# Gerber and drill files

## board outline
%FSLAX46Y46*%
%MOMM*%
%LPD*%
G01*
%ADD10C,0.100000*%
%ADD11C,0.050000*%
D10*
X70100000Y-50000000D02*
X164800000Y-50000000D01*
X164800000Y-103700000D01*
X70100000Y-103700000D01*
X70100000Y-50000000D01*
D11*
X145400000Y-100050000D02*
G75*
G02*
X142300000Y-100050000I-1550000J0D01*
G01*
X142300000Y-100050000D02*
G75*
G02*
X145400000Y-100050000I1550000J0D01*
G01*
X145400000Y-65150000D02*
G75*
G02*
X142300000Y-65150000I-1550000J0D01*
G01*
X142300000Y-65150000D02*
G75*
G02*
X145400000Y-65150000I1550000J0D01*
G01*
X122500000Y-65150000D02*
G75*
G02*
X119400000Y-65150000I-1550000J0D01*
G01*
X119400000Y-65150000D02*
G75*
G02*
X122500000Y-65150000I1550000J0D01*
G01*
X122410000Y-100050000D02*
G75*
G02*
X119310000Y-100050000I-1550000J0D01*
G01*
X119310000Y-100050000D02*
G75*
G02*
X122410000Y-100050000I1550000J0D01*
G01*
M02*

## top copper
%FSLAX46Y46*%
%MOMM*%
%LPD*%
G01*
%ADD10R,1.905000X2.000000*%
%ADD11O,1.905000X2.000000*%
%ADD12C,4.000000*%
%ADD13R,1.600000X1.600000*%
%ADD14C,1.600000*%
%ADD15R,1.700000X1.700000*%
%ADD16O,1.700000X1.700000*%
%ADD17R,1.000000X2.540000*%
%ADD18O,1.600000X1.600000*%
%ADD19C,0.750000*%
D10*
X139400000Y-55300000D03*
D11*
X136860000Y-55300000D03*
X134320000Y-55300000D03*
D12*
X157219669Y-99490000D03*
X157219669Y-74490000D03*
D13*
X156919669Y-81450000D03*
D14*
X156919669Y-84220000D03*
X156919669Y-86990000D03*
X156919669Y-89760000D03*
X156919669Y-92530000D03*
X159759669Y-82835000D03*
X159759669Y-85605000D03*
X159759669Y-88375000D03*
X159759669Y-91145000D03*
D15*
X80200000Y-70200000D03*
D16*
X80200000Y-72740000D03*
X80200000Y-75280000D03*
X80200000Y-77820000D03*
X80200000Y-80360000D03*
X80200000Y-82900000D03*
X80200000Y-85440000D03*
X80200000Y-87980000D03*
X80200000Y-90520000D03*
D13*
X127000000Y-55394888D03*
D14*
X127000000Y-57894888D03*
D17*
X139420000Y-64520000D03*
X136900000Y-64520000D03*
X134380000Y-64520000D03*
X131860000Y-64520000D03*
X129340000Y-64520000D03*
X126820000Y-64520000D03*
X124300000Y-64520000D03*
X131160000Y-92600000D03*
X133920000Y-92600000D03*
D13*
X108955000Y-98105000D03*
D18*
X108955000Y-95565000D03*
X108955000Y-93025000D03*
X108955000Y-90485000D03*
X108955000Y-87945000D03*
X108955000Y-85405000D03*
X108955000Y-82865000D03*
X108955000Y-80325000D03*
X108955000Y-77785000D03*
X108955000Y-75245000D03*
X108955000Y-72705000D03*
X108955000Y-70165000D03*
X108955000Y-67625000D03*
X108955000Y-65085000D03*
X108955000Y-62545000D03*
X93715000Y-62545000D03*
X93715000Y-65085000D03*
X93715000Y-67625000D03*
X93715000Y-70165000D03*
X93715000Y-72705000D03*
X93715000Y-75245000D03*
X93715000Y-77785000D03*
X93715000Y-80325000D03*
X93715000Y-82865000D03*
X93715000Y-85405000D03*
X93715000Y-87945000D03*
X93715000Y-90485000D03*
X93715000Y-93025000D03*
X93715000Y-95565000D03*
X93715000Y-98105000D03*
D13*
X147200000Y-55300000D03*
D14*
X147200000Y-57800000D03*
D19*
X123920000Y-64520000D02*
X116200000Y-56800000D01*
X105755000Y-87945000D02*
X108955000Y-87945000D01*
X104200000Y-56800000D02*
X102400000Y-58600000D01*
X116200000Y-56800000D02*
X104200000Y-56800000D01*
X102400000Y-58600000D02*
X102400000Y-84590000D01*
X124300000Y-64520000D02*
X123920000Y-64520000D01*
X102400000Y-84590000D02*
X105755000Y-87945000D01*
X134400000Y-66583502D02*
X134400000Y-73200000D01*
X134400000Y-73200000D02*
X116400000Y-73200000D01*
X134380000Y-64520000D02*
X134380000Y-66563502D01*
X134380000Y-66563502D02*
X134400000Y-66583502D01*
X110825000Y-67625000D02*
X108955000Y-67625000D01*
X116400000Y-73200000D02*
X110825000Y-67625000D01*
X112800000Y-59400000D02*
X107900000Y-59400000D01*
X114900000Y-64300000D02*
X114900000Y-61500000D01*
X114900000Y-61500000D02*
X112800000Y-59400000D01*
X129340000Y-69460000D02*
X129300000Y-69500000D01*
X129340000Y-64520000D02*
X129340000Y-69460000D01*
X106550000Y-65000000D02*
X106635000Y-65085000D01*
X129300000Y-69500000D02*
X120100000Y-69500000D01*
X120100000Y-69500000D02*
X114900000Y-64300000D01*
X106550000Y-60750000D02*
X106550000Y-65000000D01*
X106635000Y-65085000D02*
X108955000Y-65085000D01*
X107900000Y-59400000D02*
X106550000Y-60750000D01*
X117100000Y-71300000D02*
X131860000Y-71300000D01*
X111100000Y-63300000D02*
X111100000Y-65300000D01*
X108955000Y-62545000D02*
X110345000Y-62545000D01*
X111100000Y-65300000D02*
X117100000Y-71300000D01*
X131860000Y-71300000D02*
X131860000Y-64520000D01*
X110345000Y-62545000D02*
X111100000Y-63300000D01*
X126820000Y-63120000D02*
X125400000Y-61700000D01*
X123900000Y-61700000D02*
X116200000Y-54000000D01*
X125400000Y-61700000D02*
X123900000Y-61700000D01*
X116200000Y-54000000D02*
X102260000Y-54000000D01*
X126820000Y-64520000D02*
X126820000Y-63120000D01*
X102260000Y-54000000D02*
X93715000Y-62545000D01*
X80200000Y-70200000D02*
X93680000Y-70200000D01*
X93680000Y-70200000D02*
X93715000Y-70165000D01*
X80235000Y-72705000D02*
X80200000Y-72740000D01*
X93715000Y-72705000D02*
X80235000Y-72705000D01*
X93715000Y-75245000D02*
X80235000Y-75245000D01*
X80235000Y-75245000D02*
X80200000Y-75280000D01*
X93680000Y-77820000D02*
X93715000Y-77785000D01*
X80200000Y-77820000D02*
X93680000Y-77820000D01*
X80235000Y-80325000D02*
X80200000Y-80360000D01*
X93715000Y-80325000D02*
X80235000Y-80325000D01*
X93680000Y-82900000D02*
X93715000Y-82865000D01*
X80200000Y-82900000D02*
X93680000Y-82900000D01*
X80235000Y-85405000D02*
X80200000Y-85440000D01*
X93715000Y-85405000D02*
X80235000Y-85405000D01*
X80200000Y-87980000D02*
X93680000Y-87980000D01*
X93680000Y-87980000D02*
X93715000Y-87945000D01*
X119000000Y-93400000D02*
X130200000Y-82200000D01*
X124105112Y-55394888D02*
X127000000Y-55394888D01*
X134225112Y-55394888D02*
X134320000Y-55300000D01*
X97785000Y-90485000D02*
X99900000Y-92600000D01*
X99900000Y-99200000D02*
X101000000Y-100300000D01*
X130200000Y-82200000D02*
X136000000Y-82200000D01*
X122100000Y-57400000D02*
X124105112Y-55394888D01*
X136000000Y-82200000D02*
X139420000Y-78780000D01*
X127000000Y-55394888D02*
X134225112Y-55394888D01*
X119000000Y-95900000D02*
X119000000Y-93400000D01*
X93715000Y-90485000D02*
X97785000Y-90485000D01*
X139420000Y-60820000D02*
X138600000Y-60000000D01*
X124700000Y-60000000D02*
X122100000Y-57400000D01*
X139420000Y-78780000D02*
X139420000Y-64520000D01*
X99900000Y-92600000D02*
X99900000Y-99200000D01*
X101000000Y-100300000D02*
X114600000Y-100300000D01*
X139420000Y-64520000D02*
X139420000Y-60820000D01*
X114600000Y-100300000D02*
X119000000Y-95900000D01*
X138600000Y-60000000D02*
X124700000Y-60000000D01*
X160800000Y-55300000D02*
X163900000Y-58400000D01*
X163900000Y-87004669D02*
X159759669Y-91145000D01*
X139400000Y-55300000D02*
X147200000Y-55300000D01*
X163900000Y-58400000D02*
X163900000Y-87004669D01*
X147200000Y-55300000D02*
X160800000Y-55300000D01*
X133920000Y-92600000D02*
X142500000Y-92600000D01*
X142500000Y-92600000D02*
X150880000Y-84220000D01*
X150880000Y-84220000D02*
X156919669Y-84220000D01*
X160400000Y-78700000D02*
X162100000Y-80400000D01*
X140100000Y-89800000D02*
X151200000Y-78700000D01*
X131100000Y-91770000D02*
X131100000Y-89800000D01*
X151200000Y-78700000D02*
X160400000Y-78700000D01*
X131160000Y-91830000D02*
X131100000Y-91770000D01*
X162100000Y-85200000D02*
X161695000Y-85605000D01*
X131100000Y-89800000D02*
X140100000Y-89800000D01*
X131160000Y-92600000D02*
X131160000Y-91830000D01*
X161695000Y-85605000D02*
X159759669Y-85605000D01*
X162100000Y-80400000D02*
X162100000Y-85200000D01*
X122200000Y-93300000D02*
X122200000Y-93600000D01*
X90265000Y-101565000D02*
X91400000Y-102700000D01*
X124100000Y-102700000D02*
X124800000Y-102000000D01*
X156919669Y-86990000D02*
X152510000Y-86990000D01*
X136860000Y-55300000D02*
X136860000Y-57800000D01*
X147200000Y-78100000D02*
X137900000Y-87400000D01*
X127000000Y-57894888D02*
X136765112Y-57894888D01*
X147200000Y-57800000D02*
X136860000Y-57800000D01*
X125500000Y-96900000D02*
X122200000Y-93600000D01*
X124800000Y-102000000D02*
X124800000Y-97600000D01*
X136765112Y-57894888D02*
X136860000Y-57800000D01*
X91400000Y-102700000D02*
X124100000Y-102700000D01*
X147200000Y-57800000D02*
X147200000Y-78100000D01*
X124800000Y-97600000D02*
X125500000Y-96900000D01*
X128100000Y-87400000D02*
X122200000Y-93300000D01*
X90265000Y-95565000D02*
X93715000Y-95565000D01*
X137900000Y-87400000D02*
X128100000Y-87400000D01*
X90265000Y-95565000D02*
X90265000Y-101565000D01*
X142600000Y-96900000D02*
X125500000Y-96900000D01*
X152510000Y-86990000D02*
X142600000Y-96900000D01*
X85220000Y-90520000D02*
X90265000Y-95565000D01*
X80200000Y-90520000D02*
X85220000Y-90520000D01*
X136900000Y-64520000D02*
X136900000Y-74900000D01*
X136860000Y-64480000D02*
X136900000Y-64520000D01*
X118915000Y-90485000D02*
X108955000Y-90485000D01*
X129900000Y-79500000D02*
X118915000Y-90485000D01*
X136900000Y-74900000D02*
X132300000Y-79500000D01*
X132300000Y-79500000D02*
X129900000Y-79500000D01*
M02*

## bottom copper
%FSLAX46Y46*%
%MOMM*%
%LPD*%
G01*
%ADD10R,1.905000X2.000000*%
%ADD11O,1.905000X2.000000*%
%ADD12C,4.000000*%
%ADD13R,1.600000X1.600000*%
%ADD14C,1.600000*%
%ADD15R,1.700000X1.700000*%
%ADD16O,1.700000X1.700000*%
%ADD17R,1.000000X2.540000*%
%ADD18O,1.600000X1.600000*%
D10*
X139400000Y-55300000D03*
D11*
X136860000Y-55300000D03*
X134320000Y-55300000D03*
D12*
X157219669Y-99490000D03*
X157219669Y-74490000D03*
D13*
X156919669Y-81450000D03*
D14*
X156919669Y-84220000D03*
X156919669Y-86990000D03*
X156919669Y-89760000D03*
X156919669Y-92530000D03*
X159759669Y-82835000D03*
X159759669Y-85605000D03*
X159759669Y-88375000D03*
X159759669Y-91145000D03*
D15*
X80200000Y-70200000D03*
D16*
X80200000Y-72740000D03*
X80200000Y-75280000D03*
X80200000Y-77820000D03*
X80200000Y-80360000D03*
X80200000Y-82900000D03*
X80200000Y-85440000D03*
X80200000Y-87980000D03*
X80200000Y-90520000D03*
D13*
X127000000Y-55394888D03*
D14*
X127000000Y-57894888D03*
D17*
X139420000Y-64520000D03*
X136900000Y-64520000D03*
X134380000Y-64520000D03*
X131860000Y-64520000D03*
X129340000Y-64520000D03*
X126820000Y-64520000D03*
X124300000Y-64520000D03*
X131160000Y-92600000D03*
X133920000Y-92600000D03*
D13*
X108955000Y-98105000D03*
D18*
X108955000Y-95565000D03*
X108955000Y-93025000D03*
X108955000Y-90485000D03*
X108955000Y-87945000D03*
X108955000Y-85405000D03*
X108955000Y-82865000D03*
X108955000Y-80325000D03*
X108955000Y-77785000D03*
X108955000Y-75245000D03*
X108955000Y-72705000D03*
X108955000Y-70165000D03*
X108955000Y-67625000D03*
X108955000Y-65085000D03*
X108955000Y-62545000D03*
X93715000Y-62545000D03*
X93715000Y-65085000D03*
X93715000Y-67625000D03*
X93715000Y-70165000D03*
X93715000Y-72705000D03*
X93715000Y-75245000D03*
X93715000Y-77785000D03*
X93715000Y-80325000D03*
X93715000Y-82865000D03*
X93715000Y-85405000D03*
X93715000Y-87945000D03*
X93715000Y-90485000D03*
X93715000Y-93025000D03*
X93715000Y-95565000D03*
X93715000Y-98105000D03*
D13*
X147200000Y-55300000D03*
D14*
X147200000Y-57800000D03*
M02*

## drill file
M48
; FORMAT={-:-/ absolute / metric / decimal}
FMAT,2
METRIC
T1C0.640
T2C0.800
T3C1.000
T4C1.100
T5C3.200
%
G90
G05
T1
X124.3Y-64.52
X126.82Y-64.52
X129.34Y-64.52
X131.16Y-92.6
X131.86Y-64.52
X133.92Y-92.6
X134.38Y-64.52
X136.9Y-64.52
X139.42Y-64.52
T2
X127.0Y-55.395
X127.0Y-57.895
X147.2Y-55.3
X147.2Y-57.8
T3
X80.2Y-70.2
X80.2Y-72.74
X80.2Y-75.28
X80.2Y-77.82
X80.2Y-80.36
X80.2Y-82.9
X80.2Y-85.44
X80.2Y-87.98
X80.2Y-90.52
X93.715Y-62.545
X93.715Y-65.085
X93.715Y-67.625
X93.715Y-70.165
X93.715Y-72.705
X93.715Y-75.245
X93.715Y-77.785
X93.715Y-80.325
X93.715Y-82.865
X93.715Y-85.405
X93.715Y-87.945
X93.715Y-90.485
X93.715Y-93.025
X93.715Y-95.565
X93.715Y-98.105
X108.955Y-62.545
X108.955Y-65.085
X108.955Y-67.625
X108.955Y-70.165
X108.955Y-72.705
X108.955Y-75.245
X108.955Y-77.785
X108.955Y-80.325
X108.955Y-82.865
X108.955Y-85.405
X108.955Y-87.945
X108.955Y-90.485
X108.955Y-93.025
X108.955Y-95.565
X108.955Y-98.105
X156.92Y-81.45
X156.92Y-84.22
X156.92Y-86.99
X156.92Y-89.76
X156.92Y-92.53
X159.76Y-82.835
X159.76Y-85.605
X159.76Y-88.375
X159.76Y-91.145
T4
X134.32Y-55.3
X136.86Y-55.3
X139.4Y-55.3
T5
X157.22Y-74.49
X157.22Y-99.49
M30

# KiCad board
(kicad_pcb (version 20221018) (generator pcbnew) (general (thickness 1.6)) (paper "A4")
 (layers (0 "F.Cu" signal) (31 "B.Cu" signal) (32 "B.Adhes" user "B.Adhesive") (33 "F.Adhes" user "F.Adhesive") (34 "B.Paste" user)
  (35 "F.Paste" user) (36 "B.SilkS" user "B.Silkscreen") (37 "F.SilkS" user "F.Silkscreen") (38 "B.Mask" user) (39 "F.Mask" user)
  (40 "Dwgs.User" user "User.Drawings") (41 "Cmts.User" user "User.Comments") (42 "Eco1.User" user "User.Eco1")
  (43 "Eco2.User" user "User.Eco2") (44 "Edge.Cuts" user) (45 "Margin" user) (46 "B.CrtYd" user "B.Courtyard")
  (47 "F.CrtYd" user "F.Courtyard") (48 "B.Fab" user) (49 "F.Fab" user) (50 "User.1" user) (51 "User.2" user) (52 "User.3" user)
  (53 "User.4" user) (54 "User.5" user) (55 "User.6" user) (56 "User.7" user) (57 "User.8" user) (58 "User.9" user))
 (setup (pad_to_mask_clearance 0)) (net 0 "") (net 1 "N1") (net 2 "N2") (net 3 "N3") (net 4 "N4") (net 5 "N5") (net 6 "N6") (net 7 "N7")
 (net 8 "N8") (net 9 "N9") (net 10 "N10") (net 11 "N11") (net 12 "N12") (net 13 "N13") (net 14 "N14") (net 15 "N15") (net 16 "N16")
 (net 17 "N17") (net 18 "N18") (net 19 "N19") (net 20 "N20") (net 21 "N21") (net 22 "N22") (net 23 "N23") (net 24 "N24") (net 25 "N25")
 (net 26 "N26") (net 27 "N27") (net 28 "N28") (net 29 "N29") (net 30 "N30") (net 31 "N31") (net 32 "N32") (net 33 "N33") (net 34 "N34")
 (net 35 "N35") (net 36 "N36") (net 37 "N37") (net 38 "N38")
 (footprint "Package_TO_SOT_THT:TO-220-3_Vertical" (layer "F.Cu") (at 139.4 55.3 180)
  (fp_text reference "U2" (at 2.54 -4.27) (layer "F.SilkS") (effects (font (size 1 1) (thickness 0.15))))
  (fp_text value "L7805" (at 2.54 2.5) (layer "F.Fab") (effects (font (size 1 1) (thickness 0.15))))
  (pad "1" thru_hole rect (at 0 0 180) (size 1.905 2) (drill 1.1) (layers "*.Cu" "*.Mask") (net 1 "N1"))
  (pad "2" thru_hole oval (at 2.54 0 180) (size 1.905 2) (drill 1.1) (layers "*.Cu" "*.Mask") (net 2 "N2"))
  (pad "3" thru_hole oval (at 5.08 0 180) (size 1.905 2) (drill 1.1) (layers "*.Cu" "*.Mask") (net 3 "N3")))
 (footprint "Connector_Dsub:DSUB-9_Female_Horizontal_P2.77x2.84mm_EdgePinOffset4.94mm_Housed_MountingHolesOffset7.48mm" (layer "F.Cu")
  (at 156.919669 81.45 90)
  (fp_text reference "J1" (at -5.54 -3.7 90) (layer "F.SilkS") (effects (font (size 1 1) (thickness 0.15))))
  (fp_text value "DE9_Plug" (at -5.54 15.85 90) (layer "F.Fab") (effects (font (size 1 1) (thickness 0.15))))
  (pad "0" thru_hole circle (at -18.04 0.3 90) (size 4 4) (drill 3.2) (layers "*.Cu" "*.Mask"))
  (pad "0" thru_hole circle (at 6.96 0.3 90) (size 4 4) (drill 3.2) (layers "*.Cu" "*.Mask"))
  (pad "1" thru_hole rect (at 0 0 90) (size 1.6 1.6) (drill 1) (layers "*.Cu" "*.Mask") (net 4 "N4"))
  (pad "2" thru_hole circle (at -2.77 0 90) (size 1.6 1.6) (drill 1) (layers "*.Cu" "*.Mask") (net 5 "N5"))
  (pad "3" thru_hole circle (at -5.54 0 90) (size 1.6 1.6) (drill 1) (layers "*.Cu" "*.Mask") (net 2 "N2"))
  (pad "4" thru_hole circle (at -8.31 0 90) (size 1.6 1.6) (drill 1) (layers "*.Cu" "*.Mask") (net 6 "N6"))
  (pad "5" thru_hole circle (at -11.08 0 90) (size 1.6 1.6) (drill 1) (layers "*.Cu" "*.Mask") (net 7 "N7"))
  (pad "6" thru_hole circle (at -1.385 2.84 90) (size 1.6 1.6) (drill 1) (layers "*.Cu" "*.Mask") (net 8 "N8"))
  (pad "7" thru_hole circle (at -4.155 2.84 90) (size 1.6 1.6) (drill 1) (layers "*.Cu" "*.Mask") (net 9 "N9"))
  (pad "8" thru_hole circle (at -6.925 2.84 90) (size 1.6 1.6) (drill 1) (layers "*.Cu" "*.Mask") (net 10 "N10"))
  (pad "9" thru_hole circle (at -9.695 2.84 90) (size 1.6 1.6) (drill 1) (layers "*.Cu" "*.Mask") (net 1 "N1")))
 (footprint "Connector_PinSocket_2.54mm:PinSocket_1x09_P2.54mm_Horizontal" (layer "F.Cu") (at 80.2 70.2)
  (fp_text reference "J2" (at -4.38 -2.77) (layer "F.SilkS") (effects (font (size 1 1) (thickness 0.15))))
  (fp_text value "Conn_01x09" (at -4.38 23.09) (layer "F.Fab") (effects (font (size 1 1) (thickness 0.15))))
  (pad "1" thru_hole rect (at 0 0) (size 1.7 1.7) (drill 1) (layers "*.Cu" "*.Mask") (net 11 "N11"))
  (pad "2" thru_hole oval (at 0 2.54) (size 1.7 1.7) (drill 1) (layers "*.Cu" "*.Mask") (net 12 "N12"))
  (pad "3" thru_hole oval (at 0 5.08) (size 1.7 1.7) (drill 1) (layers "*.Cu" "*.Mask") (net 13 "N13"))
  (pad "4" thru_hole oval (at 0 7.62) (size 1.7 1.7) (drill 1) (layers "*.Cu" "*.Mask") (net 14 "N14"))
  (pad "5" thru_hole oval (at 0 10.16) (size 1.7 1.7) (drill 1) (layers "*.Cu" "*.Mask") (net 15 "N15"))
  (pad "6" thru_hole oval (at 0 12.7) (size 1.7 1.7) (drill 1) (layers "*.Cu" "*.Mask") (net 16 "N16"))
  (pad "7" thru_hole oval (at 0 15.24) (size 1.7 1.7) (drill 1) (layers "*.Cu" "*.Mask") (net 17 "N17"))
  (pad "8" thru_hole oval (at 0 17.78) (size 1.7 1.7) (drill 1) (layers "*.Cu" "*.Mask") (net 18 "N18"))
  (pad "9" thru_hole oval (at 0 20.32) (size 1.7 1.7) (drill 1) (layers "*.Cu" "*.Mask") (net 2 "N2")))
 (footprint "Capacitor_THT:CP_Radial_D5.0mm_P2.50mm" (layer "F.Cu") (at 127 55.394888 -90)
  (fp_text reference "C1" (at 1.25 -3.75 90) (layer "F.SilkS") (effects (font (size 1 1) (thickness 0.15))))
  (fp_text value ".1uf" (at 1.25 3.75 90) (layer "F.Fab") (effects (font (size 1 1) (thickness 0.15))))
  (pad "1" thru_hole rect (at 0 0 270) (size 1.6 1.6) (drill 0.8) (layers "*.Cu" "*.Mask") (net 3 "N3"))
  (pad "2" thru_hole circle (at 2.5 0 270) (size 1.6 1.6) (drill 0.8) (layers "*.Cu" "*.Mask") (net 2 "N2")))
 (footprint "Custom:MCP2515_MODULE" (layer "F.Cu") (at 118.3 62.6 180) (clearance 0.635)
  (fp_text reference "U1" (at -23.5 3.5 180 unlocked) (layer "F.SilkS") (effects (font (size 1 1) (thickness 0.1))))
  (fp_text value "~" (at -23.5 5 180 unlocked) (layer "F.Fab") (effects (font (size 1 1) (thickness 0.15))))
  (fp_circle (center -25.55 -37.45) (end -24 -37.45) (stroke (width 0.05) (type default)) (fill none) (layer "Edge.Cuts"))
  (fp_circle (center -25.55 -2.55) (end -24 -2.55) (stroke (width 0.05) (type default)) (fill none) (layer "Edge.Cuts"))
  (fp_circle (center -2.65 -2.55) (end -1.1 -2.55) (stroke (width 0.05) (type default)) (fill none) (layer "Edge.Cuts"))
  (fp_circle (center -2.56 -37.45) (end -1.01 -37.45) (stroke (width 0.05) (type default)) (fill none) (layer "Edge.Cuts"))
  (pad "1" thru_hole rect (at -21.12 -1.92 180) (size 1 2.54) (drill 0.64) (layers "*.Cu" "*.Mask") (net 3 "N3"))
  (pad "2" thru_hole rect (at -18.6 -1.92 180) (size 1 2.54) (drill 0.64) (layers "*.Cu" "*.Mask") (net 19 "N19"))
  (pad "3" thru_hole rect (at -16.08 -1.92 180) (size 1 2.54) (drill 0.64) (layers "*.Cu" "*.Mask") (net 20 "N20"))
  (pad "4" thru_hole rect (at -13.56 -1.92 180) (size 1 2.54) (drill 0.64) (layers "*.Cu" "*.Mask") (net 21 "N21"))
  (pad "5" thru_hole rect (at -11.04 -1.92 180) (size 1 2.54) (drill 0.64) (layers "*.Cu" "*.Mask") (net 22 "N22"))
  (pad "6" thru_hole rect (at -8.52 -1.92 180) (size 1 2.54) (drill 0.64) (layers "*.Cu" "*.Mask") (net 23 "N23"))
  (pad "7" thru_hole rect (at -6 -1.92 180) (size 1 2.54) (drill 0.64) (layers "*.Cu" "*.Mask") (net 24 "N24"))
  (pad "8" thru_hole rect (at -12.86 -30 180) (size 1 2.54) (drill 0.64) (layers "*.Cu" "*.Mask") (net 9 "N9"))
  (pad "9" thru_hole rect (at -15.62 -30 180) (size 1 2.54) (drill 0.64) (layers "*.Cu" "*.Mask") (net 5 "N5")))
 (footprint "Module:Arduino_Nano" (layer "F.Cu") (at 108.955 98.105 180)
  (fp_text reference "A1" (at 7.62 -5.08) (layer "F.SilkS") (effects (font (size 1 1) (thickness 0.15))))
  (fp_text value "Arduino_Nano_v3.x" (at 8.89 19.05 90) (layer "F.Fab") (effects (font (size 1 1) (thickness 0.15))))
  (pad "1" thru_hole rect (at 0 0 180) (size 1.6 1.6) (drill 1) (layers "*.Cu" "*.Mask") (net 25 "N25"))
  (pad "2" thru_hole oval (at 0 2.54 180) (size 1.6 1.6) (drill 1) (layers "*.Cu" "*.Mask") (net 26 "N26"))
  (pad "3" thru_hole oval (at 0 5.08 180) (size 1.6 1.6) (drill 1) (layers "*.Cu" "*.Mask") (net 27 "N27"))
  (pad "4" thru_hole oval (at 0 7.62 180) (size 1.6 1.6) (drill 1) (layers "*.Cu" "*.Mask") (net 19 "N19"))
  (pad "5" thru_hole oval (at 0 10.16 180) (size 1.6 1.6) (drill 1) (layers "*.Cu" "*.Mask") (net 24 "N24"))
  (pad "6" thru_hole oval (at 0 12.7 180) (size 1.6 1.6) (drill 1) (layers "*.Cu" "*.Mask") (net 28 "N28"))
  (pad "7" thru_hole oval (at 0 15.24 180) (size 1.6 1.6) (drill 1) (layers "*.Cu" "*.Mask") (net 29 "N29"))
  (pad "8" thru_hole oval (at 0 17.78 180) (size 1.6 1.6) (drill 1) (layers "*.Cu" "*.Mask") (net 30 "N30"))
  (pad "9" thru_hole oval (at 0 20.32 180) (size 1.6 1.6) (drill 1) (layers "*.Cu" "*.Mask") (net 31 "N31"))
  (pad "10" thru_hole oval (at 0 22.86 180) (size 1.6 1.6) (drill 1) (layers "*.Cu" "*.Mask") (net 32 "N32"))
  (pad "11" thru_hole oval (at 0 25.4 180) (size 1.6 1.6) (drill 1) (layers "*.Cu" "*.Mask") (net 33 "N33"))
  (pad "12" thru_hole oval (at 0 27.94 180) (size 1.6 1.6) (drill 1) (layers "*.Cu" "*.Mask") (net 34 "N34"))
  (pad "13" thru_hole oval (at 0 30.48 180) (size 1.6 1.6) (drill 1) (layers "*.Cu" "*.Mask") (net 20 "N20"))
  (pad "14" thru_hole oval (at 0 33.02 180) (size 1.6 1.6) (drill 1) (layers "*.Cu" "*.Mask") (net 22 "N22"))
  (pad "15" thru_hole oval (at 0 35.56 180) (size 1.6 1.6) (drill 1) (layers "*.Cu" "*.Mask") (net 21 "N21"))
  (pad "16" thru_hole oval (at 15.24 35.56 180) (size 1.6 1.6) (drill 1) (layers "*.Cu" "*.Mask") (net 23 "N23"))
  (pad "17" thru_hole oval (at 15.24 33.02 180) (size 1.6 1.6) (drill 1) (layers "*.Cu" "*.Mask") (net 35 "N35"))
  (pad "18" thru_hole oval (at 15.24 30.48 180) (size 1.6 1.6) (drill 1) (layers "*.Cu" "*.Mask") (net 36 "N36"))
  (pad "19" thru_hole oval (at 15.24 27.94 180) (size 1.6 1.6) (drill 1) (layers "*.Cu" "*.Mask") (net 11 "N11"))
  (pad "20" thru_hole oval (at 15.24 25.4 180) (size 1.6 1.6) (drill 1) (layers "*.Cu" "*.Mask") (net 12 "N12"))
  (pad "21" thru_hole oval (at 15.24 22.86 180) (size 1.6 1.6) (drill 1) (layers "*.Cu" "*.Mask") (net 13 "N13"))
  (pad "22" thru_hole oval (at 15.24 20.32 180) (size 1.6 1.6) (drill 1) (layers "*.Cu" "*.Mask") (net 14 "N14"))
  (pad "23" thru_hole oval (at 15.24 17.78 180) (size 1.6 1.6) (drill 1) (layers "*.Cu" "*.Mask") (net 15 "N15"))
  (pad "24" thru_hole oval (at 15.24 15.24 180) (size 1.6 1.6) (drill 1) (layers "*.Cu" "*.Mask") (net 16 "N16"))
  (pad "25" thru_hole oval (at 15.24 12.7 180) (size 1.6 1.6) (drill 1) (layers "*.Cu" "*.Mask") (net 17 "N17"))
  (pad "26" thru_hole oval (at 15.24 10.16 180) (size 1.6 1.6) (drill 1) (layers "*.Cu" "*.Mask") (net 18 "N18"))
  (pad "27" thru_hole oval (at 15.24 7.62 180) (size 1.6 1.6) (drill 1) (layers "*.Cu" "*.Mask") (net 3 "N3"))
  (pad "28" thru_hole oval (at 15.24 5.08 180) (size 1.6 1.6) (drill 1) (layers "*.Cu" "*.Mask") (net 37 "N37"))
  (pad "29" thru_hole oval (at 15.24 2.54 180) (size 1.6 1.6) (drill 1) (layers "*.Cu" "*.Mask") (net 2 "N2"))
  (pad "30" thru_hole oval (at 15.24 0 180) (size 1.6 1.6) (drill 1) (layers "*.Cu" "*.Mask") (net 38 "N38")))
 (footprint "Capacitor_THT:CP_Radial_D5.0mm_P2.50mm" (layer "F.Cu") (at 147.2 55.3 -90)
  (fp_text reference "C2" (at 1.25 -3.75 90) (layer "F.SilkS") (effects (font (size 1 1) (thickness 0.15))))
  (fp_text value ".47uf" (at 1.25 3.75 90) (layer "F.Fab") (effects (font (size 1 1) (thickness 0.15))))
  (pad "1" thru_hole rect (at 0 0 270) (size 1.6 1.6) (drill 0.8) (layers "*.Cu" "*.Mask") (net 1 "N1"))
  (pad "2" thru_hole circle (at 2.5 0 270) (size 1.6 1.6) (drill 0.8) (layers "*.Cu" "*.Mask") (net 2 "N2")))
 (gr_rect (start 70.1 50) (end 164.8 103.7) (stroke (width 0.1) (type default)) (fill none) (layer "Edge.Cuts"))
 (segment (start 123.92 64.52) (end 116.2 56.8) (width 0.75) (layer "F.Cu") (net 24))
 (segment (start 105.755 87.945) (end 108.955 87.945) (width 0.75) (layer "F.Cu") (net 24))
 (segment (start 104.2 56.8) (end 102.4 58.6) (width 0.75) (layer "F.Cu") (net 24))
 (segment (start 116.2 56.8) (end 104.2 56.8) (width 0.75) (layer "F.Cu") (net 24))
 (segment (start 102.4 58.6) (end 102.4 84.59) (width 0.75) (layer "F.Cu") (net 24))
 (segment (start 124.3 64.52) (end 123.92 64.52) (width 0.75) (layer "F.Cu") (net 24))
 (segment (start 102.4 84.59) (end 105.755 87.945) (width 0.75) (layer "F.Cu") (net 24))
 (segment (start 134.4 66.583502) (end 134.4 73.2) (width 0.75) (layer "F.Cu") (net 20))
 (segment (start 134.4 73.2) (end 116.4 73.2) (width 0.75) (layer "F.Cu") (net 20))
 (segment (start 134.38 64.52) (end 134.38 66.563502) (width 0.75) (layer "F.Cu") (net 20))
 (segment (start 134.38 66.563502) (end 134.4 66.583502) (width 0.75) (layer "F.Cu") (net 20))
 (segment (start 110.825 67.625) (end 108.955 67.625) (width 0.75) (layer "F.Cu") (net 20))
 (segment (start 116.4 73.2) (end 110.825 67.625) (width 0.75) (layer "F.Cu") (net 20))
 (segment (start 112.8 59.4) (end 107.9 59.4) (width 0.75) (layer "F.Cu") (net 22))
 (segment (start 114.9 64.3) (end 114.9 61.5) (width 0.75) (layer "F.Cu") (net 22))
 (segment (start 114.9 61.5) (end 112.8 59.4) (width 0.75) (layer "F.Cu") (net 22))
 (segment (start 129.34 69.46) (end 129.3 69.5) (width 0.75) (layer "F.Cu") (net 22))
 (segment (start 129.34 64.52) (end 129.34 69.46) (width 0.75) (layer "F.Cu") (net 22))
 (segment (start 106.55 65) (end 106.635 65.085) (width 0.75) (layer "F.Cu") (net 22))
 (segment (start 129.3 69.5) (end 120.1 69.5) (width 0.75) (layer "F.Cu") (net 22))
 (segment (start 120.1 69.5) (end 114.9 64.3) (width 0.75) (layer "F.Cu") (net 22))
 (segment (start 106.55 60.75) (end 106.55 65) (width 0.75) (layer "F.Cu") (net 22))
 (segment (start 106.635 65.085) (end 108.955 65.085) (width 0.75) (layer "F.Cu") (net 22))
 (segment (start 107.9 59.4) (end 106.55 60.75) (width 0.75) (layer "F.Cu") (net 22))
 (segment (start 117.1 71.3) (end 131.86 71.3) (width 0.75) (layer "F.Cu") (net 21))
 (segment (start 111.1 63.3) (end 111.1 65.3) (width 0.75) (layer "F.Cu") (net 21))
 (segment (start 108.955 62.545) (end 110.345 62.545) (width 0.75) (layer "F.Cu") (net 21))
 (segment (start 111.1 65.3) (end 117.1 71.3) (width 0.75) (layer "F.Cu") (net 21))
 (segment (start 131.86 71.3) (end 131.86 64.52) (width 0.75) (layer "F.Cu") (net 21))
 (segment (start 110.345 62.545) (end 111.1 63.3) (width 0.75) (layer "F.Cu") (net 21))
 (segment (start 126.82 63.12) (end 125.4 61.7) (width 0.75) (layer "F.Cu") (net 23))
 (segment (start 123.9 61.7) (end 116.2 54) (width 0.75) (layer "F.Cu") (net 23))
 (segment (start 125.4 61.7) (end 123.9 61.7) (width 0.75) (layer "F.Cu") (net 23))
 (segment (start 116.2 54) (end 102.26 54) (width 0.75) (layer "F.Cu") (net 23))
 (segment (start 126.82 64.52) (end 126.82 63.12) (width 0.75) (layer "F.Cu") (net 23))
 (segment (start 102.26 54) (end 93.715 62.545) (width 0.75) (layer "F.Cu") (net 23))
 (segment (start 80.2 70.2) (end 93.68 70.2) (width 0.75) (layer "F.Cu") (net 11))
 (segment (start 93.68 70.2) (end 93.715 70.165) (width 0.75) (layer "F.Cu") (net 11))
 (segment (start 80.235 72.705) (end 80.2 72.74) (width 0.75) (layer "F.Cu") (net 12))
 (segment (start 93.715 72.705) (end 80.235 72.705) (width 0.75) (layer "F.Cu") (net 12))
 (segment (start 93.715 75.245) (end 80.235 75.245) (width 0.75) (layer "F.Cu") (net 13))
 (segment (start 80.235 75.245) (end 80.2 75.28) (width 0.75) (layer "F.Cu") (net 13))
 (segment (start 93.68 77.82) (end 93.715 77.785) (width 0.75) (layer "F.Cu") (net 14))
 (segment (start 80.2 77.82) (end 93.68 77.82) (width 0.75) (layer "F.Cu") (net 14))
 (segment (start 80.235 80.325) (end 80.2 80.36) (width 0.75) (layer "F.Cu") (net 15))
 (segment (start 93.715 80.325) (end 80.235 80.325) (width 0.75) (layer "F.Cu") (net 15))
 (segment (start 93.68 82.9) (end 93.715 82.865) (width 0.75) (layer "F.Cu") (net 16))
 (segment (start 80.2 82.9) (end 93.68 82.9) (width 0.75) (layer "F.Cu") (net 16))
 (segment (start 80.235 85.405) (end 80.2 85.44) (width 0.75) (layer "F.Cu") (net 17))
 (segment (start 93.715 85.405) (end 80.235 85.405) (width 0.75) (layer "F.Cu") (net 17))
 (segment (start 80.2 87.98) (end 93.68 87.98) (width 0.75) (layer "F.Cu") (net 18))
 (segment (start 93.68 87.98) (end 93.715 87.945) (width 0.75) (layer "F.Cu") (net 18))
 (segment (start 119 93.4) (end 130.2 82.2) (width 0.75) (layer "F.Cu") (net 3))
 (segment (start 124.105112 55.394888) (end 127 55.394888) (width 0.75) (layer "F.Cu") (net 3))
 (segment (start 134.225112 55.394888) (end 134.32 55.3) (width 0.75) (layer "F.Cu") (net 3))
 (segment (start 97.785 90.485) (end 99.9 92.6) (width 0.75) (layer "F.Cu") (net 3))
 (segment (start 99.9 99.2) (end 101 100.3) (width 0.75) (layer "F.Cu") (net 3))
 (segment (start 130.2 82.2) (end 136 82.2) (width 0.75) (layer "F.Cu") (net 3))
 (segment (start 122.1 57.4) (end 124.105112 55.394888) (width 0.75) (layer "F.Cu") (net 3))
 (segment (start 136 82.2) (end 139.42 78.78) (width 0.75) (layer "F.Cu") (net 3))
 (segment (start 127 55.394888) (end 134.225112 55.394888) (width 0.75) (layer "F.Cu") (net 3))
 (segment (start 119 95.9) (end 119 93.4) (width 0.75) (layer "F.Cu") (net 3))
 (segment (start 93.715 90.485) (end 97.785 90.485) (width 0.75) (layer "F.Cu") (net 3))
 (segment (start 139.42 60.82) (end 138.6 60) (width 0.75) (layer "F.Cu") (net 3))
 (segment (start 124.7 60) (end 122.1 57.4) (width 0.75) (layer "F.Cu") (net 3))
 (segment (start 139.42 78.78) (end 139.42 64.52) (width 0.75) (layer "F.Cu") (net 3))
 (segment (start 99.9 92.6) (end 99.9 99.2) (width 0.75) (layer "F.Cu") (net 3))
 (segment (start 101 100.3) (end 114.6 100.3) (width 0.75) (layer "F.Cu") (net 3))
 (segment (start 139.42 64.52) (end 139.42 60.82) (width 0.75) (layer "F.Cu") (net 3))
 (segment (start 114.6 100.3) (end 119 95.9) (width 0.75) (layer "F.Cu") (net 3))
 (segment (start 138.6 60) (end 124.7 60) (width 0.75) (layer "F.Cu") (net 3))
 (segment (start 160.8 55.3) (end 163.9 58.4) (width 0.75) (layer "F.Cu") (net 1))
 (segment (start 163.9 87.004669) (end 159.759669 91.145) (width 0.75) (layer "F.Cu") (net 1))
 (segment (start 139.4 55.3) (end 147.2 55.3) (width 0.75) (layer "F.Cu") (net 1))
 (segment (start 163.9 58.4) (end 163.9 87.004669) (width 0.75) (layer "F.Cu") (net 1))
 (segment (start 147.2 55.3) (end 160.8 55.3) (width 0.75) (layer "F.Cu") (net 1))
 (segment (start 133.92 92.6) (end 142.5 92.6) (width 0.75) (layer "F.Cu") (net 5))
 (segment (start 142.5 92.6) (end 150.88 84.22) (width 0.75) (layer "F.Cu") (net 5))
 (segment (start 150.88 84.22) (end 156.919669 84.22) (width 0.75) (layer "F.Cu") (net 5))
 (segment (start 160.4 78.7) (end 162.1 80.4) (width 0.75) (layer "F.Cu") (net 9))
 (segment (start 140.1 89.8) (end 151.2 78.7) (width 0.75) (layer "F.Cu") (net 9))
 (segment (start 131.1 91.77) (end 131.1 89.8) (width 0.75) (layer "F.Cu") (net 9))
 (segment (start 151.2 78.7) (end 160.4 78.7) (width 0.75) (layer "F.Cu") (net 9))
 (segment (start 131.16 91.83) (end 131.1 91.77) (width 0.75) (layer "F.Cu") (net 9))
 (segment (start 162.1 85.2) (end 161.695 85.605) (width 0.75) (layer "F.Cu") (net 9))
 (segment (start 131.1 89.8) (end 140.1 89.8) (width 0.75) (layer "F.Cu") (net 9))
 (segment (start 131.16 92.6) (end 131.16 91.83) (width 0.75) (layer "F.Cu") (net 9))
 (segment (start 161.695 85.605) (end 159.759669 85.605) (width 0.75) (layer "F.Cu") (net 9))
 (segment (start 162.1 80.4) (end 162.1 85.2) (width 0.75) (layer "F.Cu") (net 9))
 (segment (start 122.2 93.3) (end 122.2 93.6) (width 0.75) (layer "F.Cu") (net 2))
 (segment (start 90.265 101.565) (end 91.4 102.7) (width 0.75) (layer "F.Cu") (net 2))
 (segment (start 124.1 102.7) (end 124.8 102) (width 0.75) (layer "F.Cu") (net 2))
 (segment (start 156.919669 86.99) (end 152.51 86.99) (width 0.75) (layer "F.Cu") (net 2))
 (segment (start 136.86 55.3) (end 136.86 57.8) (width 0.75) (layer "F.Cu") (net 2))
 (segment (start 147.2 78.1) (end 137.9 87.4) (width 0.75) (layer "F.Cu") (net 2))
 (segment (start 127 57.894888) (end 136.765112 57.894888) (width 0.75) (layer "F.Cu") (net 2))
 (segment (start 147.2 57.8) (end 136.86 57.8) (width 0.75) (layer "F.Cu") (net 2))
 (segment (start 125.5 96.9) (end 122.2 93.6) (width 0.75) (layer "F.Cu") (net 2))
 (segment (start 124.8 102) (end 124.8 97.6) (width 0.75) (layer "F.Cu") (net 2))
 (segment (start 136.765112 57.894888) (end 136.86 57.8) (width 0.75) (layer "F.Cu") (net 2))
 (segment (start 91.4 102.7) (end 124.1 102.7) (width 0.75) (layer "F.Cu") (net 2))
 (segment (start 147.2 57.8) (end 147.2 78.1) (width 0.75) (layer "F.Cu") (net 2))
 (segment (start 124.8 97.6) (end 125.5 96.9) (width 0.75) (layer "F.Cu") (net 2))
 (segment (start 128.1 87.4) (end 122.2 93.3) (width 0.75) (layer "F.Cu") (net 2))
 (segment (start 90.265 95.565) (end 93.715 95.565) (width 0.75) (layer "F.Cu") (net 2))
 (segment (start 137.9 87.4) (end 128.1 87.4) (width 0.75) (layer "F.Cu") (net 2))
 (segment (start 90.265 95.565) (end 90.265 101.565) (width 0.75) (layer "F.Cu") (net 2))
 (segment (start 142.6 96.9) (end 125.5 96.9) (width 0.75) (layer "F.Cu") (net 2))
 (segment (start 152.51 86.99) (end 142.6 96.9) (width 0.75) (layer "F.Cu") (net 2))
 (segment (start 85.22 90.52) (end 90.265 95.565) (width 0.75) (layer "F.Cu") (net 2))
 (segment (start 80.2 90.52) (end 85.22 90.52) (width 0.75) (layer "F.Cu") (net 2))
 (segment (start 136.9 64.52) (end 136.9 74.9) (width 0.75) (layer "F.Cu") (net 19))
 (segment (start 136.86 64.48) (end 136.9 64.52) (width 0.75) (layer "F.Cu") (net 19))
 (segment (start 118.915 90.485) (end 108.955 90.485) (width 0.75) (layer "F.Cu") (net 19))
 (segment (start 129.9 79.5) (end 118.915 90.485) (width 0.75) (layer "F.Cu") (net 19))
 (segment (start 136.9 74.9) (end 132.3 79.5) (width 0.75) (layer "F.Cu") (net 19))
 (segment (start 132.3 79.5) (end 129.9 79.5) (width 0.75) (layer "F.Cu") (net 19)))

